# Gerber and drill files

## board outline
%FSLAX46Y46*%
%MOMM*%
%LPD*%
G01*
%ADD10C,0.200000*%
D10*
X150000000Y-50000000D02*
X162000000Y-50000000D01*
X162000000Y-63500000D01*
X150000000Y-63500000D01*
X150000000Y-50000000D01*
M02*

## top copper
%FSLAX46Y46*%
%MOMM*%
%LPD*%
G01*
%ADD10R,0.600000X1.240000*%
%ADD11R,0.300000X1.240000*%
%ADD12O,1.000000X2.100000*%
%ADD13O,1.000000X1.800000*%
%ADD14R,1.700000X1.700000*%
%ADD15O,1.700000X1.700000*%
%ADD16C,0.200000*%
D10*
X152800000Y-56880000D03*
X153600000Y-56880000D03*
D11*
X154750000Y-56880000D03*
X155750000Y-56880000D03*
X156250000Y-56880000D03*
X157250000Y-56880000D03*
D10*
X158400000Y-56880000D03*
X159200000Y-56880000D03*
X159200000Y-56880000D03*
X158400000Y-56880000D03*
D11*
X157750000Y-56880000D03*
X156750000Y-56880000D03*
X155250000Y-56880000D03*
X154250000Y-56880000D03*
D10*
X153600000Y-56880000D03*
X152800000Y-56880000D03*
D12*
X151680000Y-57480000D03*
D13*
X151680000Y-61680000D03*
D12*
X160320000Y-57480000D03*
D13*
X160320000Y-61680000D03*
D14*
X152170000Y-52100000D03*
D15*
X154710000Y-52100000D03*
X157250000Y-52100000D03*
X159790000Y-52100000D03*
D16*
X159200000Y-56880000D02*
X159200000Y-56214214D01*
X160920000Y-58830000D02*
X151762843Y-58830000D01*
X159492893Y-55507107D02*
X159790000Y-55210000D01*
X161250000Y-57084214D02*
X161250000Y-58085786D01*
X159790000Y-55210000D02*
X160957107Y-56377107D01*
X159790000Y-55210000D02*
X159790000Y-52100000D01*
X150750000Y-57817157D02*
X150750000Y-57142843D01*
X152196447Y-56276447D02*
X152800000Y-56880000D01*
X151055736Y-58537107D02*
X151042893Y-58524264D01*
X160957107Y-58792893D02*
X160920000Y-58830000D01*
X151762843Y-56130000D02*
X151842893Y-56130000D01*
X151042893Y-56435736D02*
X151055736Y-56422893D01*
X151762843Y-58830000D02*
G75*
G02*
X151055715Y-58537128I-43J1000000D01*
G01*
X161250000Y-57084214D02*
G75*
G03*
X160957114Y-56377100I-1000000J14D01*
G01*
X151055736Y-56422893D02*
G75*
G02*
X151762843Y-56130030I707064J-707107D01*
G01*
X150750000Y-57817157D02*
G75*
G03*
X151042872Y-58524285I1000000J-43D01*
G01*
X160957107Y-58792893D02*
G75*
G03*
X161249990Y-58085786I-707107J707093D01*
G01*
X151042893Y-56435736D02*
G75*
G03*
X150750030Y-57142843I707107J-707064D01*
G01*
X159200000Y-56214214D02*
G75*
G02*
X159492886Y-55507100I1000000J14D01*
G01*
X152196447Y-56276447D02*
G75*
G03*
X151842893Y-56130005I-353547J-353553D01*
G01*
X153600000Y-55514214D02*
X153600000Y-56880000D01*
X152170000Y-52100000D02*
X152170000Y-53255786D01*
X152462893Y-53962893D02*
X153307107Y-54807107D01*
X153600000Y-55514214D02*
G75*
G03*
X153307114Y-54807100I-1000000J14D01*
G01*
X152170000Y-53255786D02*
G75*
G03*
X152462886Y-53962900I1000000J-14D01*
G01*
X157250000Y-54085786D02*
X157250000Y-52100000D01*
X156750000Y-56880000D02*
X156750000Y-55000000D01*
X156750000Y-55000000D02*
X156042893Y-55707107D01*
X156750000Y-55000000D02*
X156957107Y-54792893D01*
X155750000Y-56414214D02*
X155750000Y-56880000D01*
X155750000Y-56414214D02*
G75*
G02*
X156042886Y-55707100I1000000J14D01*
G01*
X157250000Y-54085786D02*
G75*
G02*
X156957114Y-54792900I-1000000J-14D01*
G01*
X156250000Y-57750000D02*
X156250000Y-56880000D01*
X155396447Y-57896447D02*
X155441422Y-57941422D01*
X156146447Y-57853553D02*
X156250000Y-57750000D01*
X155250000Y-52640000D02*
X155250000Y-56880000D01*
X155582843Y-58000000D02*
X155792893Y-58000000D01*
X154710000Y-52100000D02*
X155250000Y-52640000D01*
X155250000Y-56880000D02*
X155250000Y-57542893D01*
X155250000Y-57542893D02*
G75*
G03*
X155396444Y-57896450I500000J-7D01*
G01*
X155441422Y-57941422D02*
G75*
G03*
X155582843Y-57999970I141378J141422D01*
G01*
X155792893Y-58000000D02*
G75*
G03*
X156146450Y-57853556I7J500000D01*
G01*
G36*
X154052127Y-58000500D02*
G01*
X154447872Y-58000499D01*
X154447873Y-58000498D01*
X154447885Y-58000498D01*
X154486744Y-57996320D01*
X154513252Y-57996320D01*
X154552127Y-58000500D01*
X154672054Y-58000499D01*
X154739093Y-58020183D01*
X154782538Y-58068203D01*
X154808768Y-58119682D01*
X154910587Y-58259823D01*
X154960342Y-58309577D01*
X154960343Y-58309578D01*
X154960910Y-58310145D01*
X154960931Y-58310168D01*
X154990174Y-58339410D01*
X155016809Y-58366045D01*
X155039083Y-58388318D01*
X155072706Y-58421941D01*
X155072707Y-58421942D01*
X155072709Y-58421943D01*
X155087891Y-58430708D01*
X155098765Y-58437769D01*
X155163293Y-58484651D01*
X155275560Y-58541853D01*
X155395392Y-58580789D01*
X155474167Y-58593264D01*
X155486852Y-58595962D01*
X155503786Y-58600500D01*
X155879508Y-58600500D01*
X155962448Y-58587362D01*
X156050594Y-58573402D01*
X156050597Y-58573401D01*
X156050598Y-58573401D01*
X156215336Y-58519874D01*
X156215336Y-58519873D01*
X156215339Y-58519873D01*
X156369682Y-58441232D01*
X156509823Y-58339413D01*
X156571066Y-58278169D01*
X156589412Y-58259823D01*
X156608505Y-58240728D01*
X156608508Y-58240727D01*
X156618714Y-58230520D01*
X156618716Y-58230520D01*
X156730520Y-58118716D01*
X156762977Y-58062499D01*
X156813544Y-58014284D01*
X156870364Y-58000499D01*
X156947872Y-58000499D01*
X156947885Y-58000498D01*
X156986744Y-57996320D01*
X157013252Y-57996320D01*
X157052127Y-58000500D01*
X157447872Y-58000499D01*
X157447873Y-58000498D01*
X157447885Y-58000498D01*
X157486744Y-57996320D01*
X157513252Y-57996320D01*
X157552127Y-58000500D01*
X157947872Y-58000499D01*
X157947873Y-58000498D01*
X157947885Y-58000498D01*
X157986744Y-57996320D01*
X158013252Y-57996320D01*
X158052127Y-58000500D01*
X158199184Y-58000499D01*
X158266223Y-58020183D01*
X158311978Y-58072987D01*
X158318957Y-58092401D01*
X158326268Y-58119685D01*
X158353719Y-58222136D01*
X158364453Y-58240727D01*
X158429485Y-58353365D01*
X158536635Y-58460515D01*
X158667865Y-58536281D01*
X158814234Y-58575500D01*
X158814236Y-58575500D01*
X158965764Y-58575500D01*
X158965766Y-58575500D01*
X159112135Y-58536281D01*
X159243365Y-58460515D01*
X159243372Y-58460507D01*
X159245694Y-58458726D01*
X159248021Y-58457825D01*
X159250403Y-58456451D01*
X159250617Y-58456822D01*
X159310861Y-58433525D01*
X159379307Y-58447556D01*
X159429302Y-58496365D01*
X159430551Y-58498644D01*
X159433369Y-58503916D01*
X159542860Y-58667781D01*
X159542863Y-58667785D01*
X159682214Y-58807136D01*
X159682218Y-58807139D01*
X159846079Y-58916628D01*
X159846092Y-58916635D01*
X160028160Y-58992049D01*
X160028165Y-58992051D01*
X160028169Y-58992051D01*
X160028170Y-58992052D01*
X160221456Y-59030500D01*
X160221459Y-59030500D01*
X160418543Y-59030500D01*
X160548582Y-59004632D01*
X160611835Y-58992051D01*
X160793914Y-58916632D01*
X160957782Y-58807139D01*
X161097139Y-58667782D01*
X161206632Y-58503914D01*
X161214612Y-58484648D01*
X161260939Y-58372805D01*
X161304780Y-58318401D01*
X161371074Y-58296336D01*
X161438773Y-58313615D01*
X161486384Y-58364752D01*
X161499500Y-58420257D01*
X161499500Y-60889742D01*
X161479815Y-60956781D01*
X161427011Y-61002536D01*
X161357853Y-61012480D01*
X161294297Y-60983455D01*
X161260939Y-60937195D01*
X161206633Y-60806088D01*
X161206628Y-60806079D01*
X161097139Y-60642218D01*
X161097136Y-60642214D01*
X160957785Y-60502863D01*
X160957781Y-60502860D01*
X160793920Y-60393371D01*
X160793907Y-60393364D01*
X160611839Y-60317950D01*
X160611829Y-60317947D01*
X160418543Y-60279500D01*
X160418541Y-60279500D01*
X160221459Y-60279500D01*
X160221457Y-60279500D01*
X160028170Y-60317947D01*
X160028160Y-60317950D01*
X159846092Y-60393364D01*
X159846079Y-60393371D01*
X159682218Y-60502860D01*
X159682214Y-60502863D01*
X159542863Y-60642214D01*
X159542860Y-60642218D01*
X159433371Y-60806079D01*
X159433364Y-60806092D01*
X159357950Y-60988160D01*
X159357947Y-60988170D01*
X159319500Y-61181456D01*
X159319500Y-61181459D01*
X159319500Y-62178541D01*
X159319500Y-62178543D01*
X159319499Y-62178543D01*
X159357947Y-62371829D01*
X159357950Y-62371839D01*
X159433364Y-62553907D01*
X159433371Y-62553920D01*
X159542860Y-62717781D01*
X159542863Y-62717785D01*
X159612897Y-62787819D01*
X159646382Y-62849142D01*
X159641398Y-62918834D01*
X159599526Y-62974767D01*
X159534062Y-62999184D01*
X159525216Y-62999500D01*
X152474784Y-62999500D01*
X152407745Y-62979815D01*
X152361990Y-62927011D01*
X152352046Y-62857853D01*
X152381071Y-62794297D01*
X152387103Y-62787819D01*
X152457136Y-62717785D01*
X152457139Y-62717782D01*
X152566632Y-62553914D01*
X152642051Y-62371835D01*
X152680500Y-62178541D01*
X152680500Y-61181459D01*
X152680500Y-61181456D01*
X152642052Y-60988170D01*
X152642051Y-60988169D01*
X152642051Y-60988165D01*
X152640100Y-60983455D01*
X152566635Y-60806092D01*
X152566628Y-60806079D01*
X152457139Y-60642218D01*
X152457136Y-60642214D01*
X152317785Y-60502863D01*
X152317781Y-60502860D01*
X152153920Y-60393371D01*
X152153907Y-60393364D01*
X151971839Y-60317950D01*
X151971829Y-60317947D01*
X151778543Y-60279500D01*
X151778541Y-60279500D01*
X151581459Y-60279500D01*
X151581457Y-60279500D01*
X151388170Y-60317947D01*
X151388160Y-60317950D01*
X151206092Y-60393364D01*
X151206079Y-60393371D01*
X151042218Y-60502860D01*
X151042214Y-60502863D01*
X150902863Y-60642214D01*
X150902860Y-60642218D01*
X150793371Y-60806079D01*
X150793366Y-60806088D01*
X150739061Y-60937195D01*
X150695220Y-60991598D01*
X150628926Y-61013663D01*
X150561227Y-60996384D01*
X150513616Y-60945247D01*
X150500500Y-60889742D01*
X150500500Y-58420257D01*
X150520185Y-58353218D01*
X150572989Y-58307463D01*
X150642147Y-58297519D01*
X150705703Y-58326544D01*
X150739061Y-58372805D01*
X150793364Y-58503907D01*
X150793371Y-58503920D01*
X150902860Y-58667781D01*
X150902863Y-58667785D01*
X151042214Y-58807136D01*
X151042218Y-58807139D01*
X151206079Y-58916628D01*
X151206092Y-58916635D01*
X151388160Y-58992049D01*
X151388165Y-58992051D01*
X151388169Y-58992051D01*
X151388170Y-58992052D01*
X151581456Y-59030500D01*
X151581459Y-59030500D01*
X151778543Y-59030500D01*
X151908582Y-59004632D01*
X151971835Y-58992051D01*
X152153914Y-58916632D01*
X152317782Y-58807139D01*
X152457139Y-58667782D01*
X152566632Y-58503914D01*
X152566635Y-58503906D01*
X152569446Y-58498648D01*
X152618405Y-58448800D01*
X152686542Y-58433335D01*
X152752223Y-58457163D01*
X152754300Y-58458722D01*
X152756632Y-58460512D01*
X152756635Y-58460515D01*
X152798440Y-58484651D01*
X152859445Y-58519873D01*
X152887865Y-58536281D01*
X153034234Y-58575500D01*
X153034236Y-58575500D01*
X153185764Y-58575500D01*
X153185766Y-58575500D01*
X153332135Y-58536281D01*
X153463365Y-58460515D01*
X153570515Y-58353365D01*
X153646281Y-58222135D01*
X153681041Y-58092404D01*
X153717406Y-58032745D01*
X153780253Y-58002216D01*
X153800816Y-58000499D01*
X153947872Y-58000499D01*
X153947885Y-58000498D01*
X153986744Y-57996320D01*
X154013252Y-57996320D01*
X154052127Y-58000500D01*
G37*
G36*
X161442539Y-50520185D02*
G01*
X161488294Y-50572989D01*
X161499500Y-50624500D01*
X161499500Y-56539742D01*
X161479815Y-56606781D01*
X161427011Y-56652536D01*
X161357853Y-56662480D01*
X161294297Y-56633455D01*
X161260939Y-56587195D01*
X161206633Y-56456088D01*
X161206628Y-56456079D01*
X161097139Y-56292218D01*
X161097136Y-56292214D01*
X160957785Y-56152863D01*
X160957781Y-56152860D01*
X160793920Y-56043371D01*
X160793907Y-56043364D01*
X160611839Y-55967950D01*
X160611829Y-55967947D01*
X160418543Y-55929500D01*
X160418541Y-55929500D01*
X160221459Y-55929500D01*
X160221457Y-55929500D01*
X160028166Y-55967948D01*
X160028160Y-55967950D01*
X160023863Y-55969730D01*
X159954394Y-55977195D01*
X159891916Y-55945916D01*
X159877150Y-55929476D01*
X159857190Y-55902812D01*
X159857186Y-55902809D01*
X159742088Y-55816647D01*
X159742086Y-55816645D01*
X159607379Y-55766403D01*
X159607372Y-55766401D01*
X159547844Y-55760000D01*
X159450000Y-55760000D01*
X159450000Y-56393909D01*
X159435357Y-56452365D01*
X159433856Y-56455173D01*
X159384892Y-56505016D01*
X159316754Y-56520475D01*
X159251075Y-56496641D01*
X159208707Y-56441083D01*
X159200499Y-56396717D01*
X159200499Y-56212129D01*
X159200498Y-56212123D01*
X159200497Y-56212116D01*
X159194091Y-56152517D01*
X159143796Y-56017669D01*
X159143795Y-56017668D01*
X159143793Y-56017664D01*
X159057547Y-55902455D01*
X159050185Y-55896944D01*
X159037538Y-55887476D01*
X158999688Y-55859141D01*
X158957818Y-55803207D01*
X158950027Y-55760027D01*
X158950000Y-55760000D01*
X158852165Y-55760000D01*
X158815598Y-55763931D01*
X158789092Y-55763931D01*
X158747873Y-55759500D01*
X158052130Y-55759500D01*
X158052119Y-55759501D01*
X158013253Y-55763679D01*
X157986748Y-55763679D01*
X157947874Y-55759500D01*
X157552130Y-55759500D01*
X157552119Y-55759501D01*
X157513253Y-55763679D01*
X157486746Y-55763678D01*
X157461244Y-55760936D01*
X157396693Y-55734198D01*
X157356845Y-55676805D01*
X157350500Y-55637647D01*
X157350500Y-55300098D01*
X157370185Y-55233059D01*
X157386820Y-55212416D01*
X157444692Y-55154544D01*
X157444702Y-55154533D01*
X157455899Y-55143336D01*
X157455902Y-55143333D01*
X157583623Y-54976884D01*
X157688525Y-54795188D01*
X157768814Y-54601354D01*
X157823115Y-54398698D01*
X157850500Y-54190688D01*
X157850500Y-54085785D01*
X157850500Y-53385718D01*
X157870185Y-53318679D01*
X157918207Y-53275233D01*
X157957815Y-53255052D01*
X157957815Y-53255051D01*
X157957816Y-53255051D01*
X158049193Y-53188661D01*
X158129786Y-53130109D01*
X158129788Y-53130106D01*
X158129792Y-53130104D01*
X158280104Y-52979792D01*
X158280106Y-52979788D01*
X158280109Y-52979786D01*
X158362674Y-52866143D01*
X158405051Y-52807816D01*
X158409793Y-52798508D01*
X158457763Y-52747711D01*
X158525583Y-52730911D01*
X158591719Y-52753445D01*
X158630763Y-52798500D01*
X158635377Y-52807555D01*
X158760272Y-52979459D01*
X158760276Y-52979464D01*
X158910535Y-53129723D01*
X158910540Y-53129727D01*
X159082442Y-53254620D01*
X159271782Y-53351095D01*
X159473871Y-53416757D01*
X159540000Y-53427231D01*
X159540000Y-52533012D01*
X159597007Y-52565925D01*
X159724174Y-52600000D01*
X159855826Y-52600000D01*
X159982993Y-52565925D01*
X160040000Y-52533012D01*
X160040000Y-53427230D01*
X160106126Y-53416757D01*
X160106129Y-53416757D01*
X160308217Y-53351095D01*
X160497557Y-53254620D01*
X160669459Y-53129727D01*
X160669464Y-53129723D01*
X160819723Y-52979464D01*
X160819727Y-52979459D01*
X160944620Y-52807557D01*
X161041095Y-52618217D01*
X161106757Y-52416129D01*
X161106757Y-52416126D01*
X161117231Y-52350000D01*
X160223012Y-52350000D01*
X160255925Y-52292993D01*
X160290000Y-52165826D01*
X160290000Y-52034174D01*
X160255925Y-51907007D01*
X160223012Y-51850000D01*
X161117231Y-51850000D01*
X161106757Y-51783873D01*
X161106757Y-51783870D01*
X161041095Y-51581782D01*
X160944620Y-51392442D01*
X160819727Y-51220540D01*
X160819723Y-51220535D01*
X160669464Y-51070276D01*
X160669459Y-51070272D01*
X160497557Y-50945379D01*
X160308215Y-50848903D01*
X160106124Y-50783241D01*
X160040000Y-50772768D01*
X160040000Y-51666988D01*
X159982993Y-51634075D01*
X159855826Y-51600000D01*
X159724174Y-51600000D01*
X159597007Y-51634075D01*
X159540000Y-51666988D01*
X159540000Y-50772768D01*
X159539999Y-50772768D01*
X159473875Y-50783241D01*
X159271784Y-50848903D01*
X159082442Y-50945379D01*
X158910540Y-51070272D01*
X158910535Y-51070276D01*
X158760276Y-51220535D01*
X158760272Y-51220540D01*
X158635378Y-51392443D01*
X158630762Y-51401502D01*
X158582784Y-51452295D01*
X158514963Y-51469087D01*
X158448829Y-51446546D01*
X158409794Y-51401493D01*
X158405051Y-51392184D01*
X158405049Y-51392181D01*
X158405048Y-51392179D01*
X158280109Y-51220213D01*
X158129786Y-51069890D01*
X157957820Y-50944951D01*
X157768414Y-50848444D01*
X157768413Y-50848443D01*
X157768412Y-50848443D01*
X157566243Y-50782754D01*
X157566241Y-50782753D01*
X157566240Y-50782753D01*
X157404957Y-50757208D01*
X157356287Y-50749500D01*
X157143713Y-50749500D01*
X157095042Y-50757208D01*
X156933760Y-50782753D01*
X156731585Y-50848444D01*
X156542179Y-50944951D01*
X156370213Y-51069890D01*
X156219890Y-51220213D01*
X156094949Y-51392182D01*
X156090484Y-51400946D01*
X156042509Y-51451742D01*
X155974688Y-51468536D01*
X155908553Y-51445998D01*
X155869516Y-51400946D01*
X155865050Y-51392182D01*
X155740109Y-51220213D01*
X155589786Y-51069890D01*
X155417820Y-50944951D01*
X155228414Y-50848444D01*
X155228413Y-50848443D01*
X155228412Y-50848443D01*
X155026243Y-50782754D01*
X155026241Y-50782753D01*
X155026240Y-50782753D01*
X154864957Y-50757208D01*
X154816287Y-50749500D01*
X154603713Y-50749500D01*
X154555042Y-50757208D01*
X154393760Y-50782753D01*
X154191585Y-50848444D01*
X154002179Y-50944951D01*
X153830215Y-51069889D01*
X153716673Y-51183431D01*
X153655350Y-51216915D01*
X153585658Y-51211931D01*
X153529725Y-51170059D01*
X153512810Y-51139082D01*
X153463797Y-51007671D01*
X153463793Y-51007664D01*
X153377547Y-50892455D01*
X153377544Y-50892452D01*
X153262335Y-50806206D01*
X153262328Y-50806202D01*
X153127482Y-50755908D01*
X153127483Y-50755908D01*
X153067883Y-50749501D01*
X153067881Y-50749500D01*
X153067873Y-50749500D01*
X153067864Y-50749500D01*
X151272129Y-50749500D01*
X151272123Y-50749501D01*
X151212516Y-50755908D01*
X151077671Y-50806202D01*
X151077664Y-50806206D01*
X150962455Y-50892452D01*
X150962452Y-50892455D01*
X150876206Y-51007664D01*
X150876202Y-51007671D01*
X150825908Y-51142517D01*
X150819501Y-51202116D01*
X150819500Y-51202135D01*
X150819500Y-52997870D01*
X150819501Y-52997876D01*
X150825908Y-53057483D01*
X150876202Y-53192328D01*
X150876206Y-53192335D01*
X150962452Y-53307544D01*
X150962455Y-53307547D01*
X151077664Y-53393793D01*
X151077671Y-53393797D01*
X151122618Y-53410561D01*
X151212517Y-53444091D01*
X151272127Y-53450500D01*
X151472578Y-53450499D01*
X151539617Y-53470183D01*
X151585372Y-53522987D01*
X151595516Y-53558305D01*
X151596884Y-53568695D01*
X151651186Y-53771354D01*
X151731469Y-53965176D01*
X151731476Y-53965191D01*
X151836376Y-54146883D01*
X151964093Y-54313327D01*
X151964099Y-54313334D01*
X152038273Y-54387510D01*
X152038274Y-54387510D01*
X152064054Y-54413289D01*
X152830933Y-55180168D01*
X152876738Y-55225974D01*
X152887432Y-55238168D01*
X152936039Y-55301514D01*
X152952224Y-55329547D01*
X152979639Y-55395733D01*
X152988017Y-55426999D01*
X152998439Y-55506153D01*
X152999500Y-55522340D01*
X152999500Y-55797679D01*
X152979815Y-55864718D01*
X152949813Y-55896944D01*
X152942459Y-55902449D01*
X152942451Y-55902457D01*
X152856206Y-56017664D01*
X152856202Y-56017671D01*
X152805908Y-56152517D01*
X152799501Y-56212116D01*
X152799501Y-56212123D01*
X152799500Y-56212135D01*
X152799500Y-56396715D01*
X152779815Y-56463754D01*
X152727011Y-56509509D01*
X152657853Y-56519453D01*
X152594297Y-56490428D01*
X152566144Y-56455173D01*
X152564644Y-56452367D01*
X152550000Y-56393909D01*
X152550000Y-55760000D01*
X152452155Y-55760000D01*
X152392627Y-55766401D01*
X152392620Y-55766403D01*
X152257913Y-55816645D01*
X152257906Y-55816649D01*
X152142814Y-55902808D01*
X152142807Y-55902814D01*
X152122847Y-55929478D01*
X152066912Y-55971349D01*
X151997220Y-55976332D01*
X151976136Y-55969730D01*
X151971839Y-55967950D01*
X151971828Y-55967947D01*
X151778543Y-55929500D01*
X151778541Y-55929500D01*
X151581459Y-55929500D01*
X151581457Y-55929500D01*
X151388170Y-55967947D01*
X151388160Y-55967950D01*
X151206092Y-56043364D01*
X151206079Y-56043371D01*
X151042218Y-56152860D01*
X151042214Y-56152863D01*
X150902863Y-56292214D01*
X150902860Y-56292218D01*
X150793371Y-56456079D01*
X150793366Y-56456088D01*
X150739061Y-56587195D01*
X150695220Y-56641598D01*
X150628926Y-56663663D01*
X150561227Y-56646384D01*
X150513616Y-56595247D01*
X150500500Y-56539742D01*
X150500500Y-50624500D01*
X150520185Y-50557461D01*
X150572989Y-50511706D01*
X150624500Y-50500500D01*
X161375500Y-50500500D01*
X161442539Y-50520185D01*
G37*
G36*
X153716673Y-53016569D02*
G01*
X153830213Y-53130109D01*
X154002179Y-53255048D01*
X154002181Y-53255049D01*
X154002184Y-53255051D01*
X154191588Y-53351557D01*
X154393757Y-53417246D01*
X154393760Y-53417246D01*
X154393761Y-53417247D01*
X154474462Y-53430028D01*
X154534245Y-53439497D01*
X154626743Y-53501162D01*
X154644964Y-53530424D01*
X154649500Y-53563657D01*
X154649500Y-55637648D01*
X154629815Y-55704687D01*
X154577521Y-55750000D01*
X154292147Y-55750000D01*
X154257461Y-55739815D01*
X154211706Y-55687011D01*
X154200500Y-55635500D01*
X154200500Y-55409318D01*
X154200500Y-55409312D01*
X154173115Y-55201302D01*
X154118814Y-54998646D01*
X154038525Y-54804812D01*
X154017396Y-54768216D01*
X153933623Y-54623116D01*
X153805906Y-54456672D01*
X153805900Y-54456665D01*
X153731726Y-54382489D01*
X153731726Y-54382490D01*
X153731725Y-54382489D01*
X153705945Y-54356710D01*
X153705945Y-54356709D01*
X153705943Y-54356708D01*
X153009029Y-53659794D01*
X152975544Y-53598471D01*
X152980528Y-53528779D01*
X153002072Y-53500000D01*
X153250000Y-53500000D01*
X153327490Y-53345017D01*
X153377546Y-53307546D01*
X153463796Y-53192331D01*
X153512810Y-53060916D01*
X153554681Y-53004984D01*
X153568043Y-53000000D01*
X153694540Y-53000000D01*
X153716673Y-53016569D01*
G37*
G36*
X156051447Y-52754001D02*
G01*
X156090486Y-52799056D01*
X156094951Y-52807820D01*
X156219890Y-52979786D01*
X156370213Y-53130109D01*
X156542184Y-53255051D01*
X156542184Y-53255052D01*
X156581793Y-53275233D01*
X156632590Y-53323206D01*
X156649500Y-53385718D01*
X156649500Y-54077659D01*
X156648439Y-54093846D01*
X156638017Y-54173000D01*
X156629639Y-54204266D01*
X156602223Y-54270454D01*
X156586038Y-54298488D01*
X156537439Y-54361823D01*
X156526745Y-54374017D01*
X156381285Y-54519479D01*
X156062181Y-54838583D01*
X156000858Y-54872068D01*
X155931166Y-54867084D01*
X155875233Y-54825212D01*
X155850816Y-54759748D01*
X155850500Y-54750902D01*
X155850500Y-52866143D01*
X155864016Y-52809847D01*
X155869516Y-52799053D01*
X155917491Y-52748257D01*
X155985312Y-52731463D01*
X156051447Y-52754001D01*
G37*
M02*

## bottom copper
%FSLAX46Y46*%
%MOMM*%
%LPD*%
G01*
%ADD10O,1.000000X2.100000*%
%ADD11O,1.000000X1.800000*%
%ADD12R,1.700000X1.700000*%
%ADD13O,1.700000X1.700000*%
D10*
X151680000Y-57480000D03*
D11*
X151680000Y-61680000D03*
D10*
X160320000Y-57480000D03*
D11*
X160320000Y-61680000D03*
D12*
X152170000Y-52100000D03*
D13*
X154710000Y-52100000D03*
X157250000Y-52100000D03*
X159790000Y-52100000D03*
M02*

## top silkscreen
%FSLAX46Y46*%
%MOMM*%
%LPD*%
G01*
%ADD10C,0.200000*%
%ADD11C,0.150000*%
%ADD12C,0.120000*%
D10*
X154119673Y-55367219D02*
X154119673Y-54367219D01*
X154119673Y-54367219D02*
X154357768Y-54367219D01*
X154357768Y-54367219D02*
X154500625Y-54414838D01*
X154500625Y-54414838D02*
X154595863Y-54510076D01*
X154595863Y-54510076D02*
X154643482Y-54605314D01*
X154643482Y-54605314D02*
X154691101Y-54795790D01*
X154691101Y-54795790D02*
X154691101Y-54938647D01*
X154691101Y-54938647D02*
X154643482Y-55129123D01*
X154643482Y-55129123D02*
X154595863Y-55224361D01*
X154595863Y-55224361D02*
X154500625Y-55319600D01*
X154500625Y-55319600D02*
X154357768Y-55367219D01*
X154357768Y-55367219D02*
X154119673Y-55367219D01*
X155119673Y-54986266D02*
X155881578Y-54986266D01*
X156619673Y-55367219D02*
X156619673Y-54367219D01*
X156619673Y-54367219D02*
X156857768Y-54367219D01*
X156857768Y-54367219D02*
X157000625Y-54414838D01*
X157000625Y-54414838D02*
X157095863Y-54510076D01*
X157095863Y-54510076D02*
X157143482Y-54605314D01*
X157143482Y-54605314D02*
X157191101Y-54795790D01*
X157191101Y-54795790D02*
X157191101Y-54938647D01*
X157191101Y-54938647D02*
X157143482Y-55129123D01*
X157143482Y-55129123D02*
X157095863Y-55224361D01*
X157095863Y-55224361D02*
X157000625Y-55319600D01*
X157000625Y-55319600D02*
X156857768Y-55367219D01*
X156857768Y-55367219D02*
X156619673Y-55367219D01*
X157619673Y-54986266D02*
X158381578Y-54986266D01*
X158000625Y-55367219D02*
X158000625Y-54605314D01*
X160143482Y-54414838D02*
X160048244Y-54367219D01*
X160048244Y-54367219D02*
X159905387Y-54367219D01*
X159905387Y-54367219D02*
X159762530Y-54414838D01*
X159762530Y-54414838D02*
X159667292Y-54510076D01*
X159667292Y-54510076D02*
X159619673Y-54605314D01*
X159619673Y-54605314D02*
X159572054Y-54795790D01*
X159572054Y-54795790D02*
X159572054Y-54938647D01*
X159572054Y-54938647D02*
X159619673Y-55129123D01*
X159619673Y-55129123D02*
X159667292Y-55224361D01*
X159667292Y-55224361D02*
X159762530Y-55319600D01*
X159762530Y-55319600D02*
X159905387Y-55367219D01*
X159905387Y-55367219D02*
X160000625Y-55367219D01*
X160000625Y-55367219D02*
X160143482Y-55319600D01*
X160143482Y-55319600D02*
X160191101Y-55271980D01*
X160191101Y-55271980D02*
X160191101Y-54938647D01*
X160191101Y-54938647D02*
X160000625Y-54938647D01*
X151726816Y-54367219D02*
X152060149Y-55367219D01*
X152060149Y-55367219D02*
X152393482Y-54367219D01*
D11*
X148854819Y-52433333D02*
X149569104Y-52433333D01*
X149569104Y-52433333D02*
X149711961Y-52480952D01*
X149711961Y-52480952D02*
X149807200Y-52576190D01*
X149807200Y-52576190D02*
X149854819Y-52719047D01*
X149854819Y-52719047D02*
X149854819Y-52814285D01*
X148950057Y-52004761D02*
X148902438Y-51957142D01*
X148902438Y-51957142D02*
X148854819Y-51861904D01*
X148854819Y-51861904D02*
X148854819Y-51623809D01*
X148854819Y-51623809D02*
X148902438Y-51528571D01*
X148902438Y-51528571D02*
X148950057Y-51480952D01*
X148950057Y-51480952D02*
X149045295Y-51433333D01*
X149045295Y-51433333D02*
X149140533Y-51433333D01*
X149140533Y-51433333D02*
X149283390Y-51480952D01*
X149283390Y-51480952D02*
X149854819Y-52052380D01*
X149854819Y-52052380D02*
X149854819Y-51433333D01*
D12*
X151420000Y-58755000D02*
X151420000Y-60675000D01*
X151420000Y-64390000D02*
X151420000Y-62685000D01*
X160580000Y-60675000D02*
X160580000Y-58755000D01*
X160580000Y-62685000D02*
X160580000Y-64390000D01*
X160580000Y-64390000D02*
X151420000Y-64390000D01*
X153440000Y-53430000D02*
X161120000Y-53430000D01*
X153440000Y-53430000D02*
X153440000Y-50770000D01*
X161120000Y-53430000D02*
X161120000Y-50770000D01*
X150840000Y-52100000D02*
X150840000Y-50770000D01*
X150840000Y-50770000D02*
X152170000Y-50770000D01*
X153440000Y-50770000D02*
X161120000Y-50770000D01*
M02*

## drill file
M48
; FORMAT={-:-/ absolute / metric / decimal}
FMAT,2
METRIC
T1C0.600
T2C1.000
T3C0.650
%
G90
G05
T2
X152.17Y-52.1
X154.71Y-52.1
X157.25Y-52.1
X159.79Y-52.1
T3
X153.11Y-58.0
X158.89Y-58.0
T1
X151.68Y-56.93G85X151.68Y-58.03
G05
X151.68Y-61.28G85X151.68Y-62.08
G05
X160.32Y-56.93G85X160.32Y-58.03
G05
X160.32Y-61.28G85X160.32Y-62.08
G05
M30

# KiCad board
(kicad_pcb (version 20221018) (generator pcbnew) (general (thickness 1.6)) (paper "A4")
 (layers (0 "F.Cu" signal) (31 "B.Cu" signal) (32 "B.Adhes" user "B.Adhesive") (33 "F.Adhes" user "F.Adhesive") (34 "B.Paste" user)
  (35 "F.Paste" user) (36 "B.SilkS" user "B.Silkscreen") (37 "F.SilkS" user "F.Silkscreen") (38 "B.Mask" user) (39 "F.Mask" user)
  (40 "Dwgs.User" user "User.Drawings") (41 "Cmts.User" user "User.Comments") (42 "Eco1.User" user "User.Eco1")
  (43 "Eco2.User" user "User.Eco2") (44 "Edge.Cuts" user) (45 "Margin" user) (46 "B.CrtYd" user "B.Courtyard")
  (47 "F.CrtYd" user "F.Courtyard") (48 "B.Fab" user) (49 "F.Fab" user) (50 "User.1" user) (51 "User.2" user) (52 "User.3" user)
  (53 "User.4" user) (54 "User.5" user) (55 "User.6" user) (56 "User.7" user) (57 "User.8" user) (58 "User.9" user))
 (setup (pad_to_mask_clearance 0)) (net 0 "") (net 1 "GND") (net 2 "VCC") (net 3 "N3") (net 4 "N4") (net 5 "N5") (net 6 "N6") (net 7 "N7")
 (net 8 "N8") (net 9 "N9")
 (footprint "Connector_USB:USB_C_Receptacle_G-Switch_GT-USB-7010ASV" (layer "F.Cu") (at 156 60.605)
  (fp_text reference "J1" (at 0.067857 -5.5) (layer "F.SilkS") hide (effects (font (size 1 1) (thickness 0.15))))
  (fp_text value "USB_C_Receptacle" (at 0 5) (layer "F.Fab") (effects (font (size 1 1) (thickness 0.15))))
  (fp_line (start -4.58 -1.85) (end -4.58 0.07) (stroke (width 0.12) (type solid)) (layer "F.SilkS"))
  (fp_line (start -4.58 3.785) (end -4.58 2.08) (stroke (width 0.12) (type solid)) (layer "F.SilkS"))
  (fp_line (start 4.58 0.07) (end 4.58 -1.85) (stroke (width 0.12) (type solid)) (layer "F.SilkS"))
  (fp_line (start 4.58 2.08) (end 4.58 3.785) (stroke (width 0.12) (type solid)) (layer "F.SilkS"))
  (fp_line (start 4.58 3.785) (end -4.58 3.785) (stroke (width 0.12) (type solid)) (layer "F.SilkS"))
  (pad "" np_thru_hole circle (at -2.89 -2.605) (size 0.65 0.65) (drill 0.65) (layers "*.Cu" "*.Mask"))
  (pad "" np_thru_hole circle (at 2.89 -2.605) (size 0.65 0.65) (drill 0.65) (layers "*.Cu" "*.Mask"))
  (pad "A1" smd rect (at -3.2 -3.725) (size 0.6 1.24) (layers "F.Cu" "F.Paste" "F.Mask") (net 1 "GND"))
  (pad "A4" smd rect (at -2.4 -3.725) (size 0.6 1.24) (layers "F.Cu" "F.Paste" "F.Mask") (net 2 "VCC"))
  (pad "A5" smd rect (at -1.25 -3.725) (size 0.3 1.24) (layers "F.Cu" "F.Paste" "F.Mask") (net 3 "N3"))
  (pad "A6" smd rect (at -0.25 -3.725) (size 0.3 1.24) (layers "F.Cu" "F.Paste" "F.Mask") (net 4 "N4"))
  (pad "A7" smd rect (at 0.25 -3.725) (size 0.3 1.24) (layers "F.Cu" "F.Paste" "F.Mask") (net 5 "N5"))
  (pad "A8" smd rect (at 1.25 -3.725) (size 0.3 1.24) (layers "F.Cu" "F.Paste" "F.Mask") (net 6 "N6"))
  (pad "A9" smd rect (at 2.4 -3.725) (size 0.6 1.24) (layers "F.Cu" "F.Paste" "F.Mask") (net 2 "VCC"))
  (pad "A12" smd rect (at 3.2 -3.725) (size 0.6 1.24) (layers "F.Cu" "F.Paste" "F.Mask") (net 1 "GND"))
  (pad "B1" smd rect (at 3.2 -3.725) (size 0.6 1.24) (layers "F.Cu" "F.Paste" "F.Mask") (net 1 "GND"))
  (pad "B4" smd rect (at 2.4 -3.725) (size 0.6 1.24) (layers "F.Cu" "F.Paste" "F.Mask") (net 2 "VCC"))
  (pad "B5" smd rect (at 1.75 -3.725) (size 0.3 1.24) (layers "F.Cu" "F.Paste" "F.Mask") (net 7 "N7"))
  (pad "B6" smd rect (at 0.75 -3.725) (size 0.3 1.24) (layers "F.Cu" "F.Paste" "F.Mask") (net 4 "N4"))
  (pad "B7" smd rect (at -0.75 -3.725) (size 0.3 1.24) (layers "F.Cu" "F.Paste" "F.Mask") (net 5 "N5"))
  (pad "B8" smd rect (at -1.75 -3.725) (size 0.3 1.24) (layers "F.Cu" "F.Paste" "F.Mask") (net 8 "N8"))
  (pad "B9" smd rect (at -2.4 -3.725) (size 0.6 1.24) (layers "F.Cu" "F.Paste" "F.Mask") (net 2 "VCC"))
  (pad "B12" smd rect (at -3.2 -3.725) (size 0.6 1.24) (layers "F.Cu" "F.Paste" "F.Mask") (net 1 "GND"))
  (pad "S1" thru_hole oval (at -4.32 -3.125) (size 1 2.1) (drill oval 0.6 1.7) (layers "*.Cu" "*.Mask") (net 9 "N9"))
  (pad "S1" thru_hole oval (at -4.32 1.075) (size 1 1.8) (drill oval 0.6 1.4) (layers "*.Cu" "*.Mask") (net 9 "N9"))
  (pad "S1" thru_hole oval (at 4.32 -3.125) (size 1 2.1) (drill oval 0.6 1.7) (layers "*.Cu" "*.Mask") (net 9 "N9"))
  (pad "S1" thru_hole oval (at 4.32 1.075) (size 1 1.8) (drill oval 0.6 1.4) (layers "*.Cu" "*.Mask") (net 9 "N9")))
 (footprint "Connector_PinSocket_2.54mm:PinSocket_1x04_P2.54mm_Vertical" (layer "F.Cu") (at 152.17 52.1 90)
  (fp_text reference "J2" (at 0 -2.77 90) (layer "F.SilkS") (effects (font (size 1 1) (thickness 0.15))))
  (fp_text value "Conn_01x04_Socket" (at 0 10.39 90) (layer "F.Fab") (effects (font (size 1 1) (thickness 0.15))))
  (fp_line (start -1.33 1.27) (end -1.33 8.95) (stroke (width 0.12) (type solid)) (layer "F.SilkS"))
  (fp_line (start -1.33 1.27) (end 1.33 1.27) (stroke (width 0.12) (type solid)) (layer "F.SilkS"))
  (fp_line (start -1.33 8.95) (end 1.33 8.95) (stroke (width 0.12) (type solid)) (layer "F.SilkS"))
  (fp_line (start 0 -1.33) (end 1.33 -1.33) (stroke (width 0.12) (type solid)) (layer "F.SilkS"))
  (fp_line (start 1.33 -1.33) (end 1.33 0) (stroke (width 0.12) (type solid)) (layer "F.SilkS"))
  (fp_line (start 1.33 1.27) (end 1.33 8.95) (stroke (width 0.12) (type solid)) (layer "F.SilkS"))
  (pad "1" thru_hole rect (at 0 0 90) (size 1.7 1.7) (drill 1) (layers "*.Cu" "*.Mask") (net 2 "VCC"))
  (pad "2" thru_hole oval (at 0 2.54 90) (size 1.7 1.7) (drill 1) (layers "*.Cu" "*.Mask") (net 5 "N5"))
  (pad "3" thru_hole oval (at 0 5.08 90) (size 1.7 1.7) (drill 1) (layers "*.Cu" "*.Mask") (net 4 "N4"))
  (pad "4" thru_hole oval (at 0 7.62 90) (size 1.7 1.7) (drill 1) (layers "*.Cu" "*.Mask") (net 1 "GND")))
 (gr_rect locked (start 150 50) (end 162 63.5) (stroke (width 0.2) (type solid)) (fill none) (layer "Edge.Cuts"))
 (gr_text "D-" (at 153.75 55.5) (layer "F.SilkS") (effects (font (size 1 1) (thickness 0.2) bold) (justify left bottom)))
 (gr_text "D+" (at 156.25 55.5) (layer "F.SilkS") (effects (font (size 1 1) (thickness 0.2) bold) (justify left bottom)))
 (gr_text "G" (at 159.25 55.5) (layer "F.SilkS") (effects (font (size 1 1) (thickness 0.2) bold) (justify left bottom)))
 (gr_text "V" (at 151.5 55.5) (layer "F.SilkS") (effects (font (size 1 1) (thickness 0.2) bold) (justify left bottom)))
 (segment (start 159.2 56.88) (end 159.2 56.214214) (width 0.2) (layer "F.Cu") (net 1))
 (segment (start 160.92 58.83) (end 151.762843 58.83) (width 0.2) (layer "F.Cu") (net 1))
 (segment (start 159.492893 55.507107) (end 159.79 55.21) (width 0.2) (layer "F.Cu") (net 1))
 (segment (start 161.25 57.084214) (end 161.25 58.085786) (width 0.2) (layer "F.Cu") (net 1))
 (segment (start 159.79 55.21) (end 160.957107 56.377107) (width 0.2) (layer "F.Cu") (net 1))
 (segment (start 159.79 55.21) (end 159.79 52.1) (width 0.2) (layer "F.Cu") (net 1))
 (segment (start 150.75 57.817157) (end 150.75 57.142843) (width 0.2) (layer "F.Cu") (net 1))
 (segment (start 152.196447 56.276447) (end 152.8 56.88) (width 0.2) (layer "F.Cu") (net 1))
 (segment (start 151.055736 58.537107) (end 151.042893 58.524264) (width 0.2) (layer "F.Cu") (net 1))
 (segment (start 160.957107 58.792893) (end 160.92 58.83) (width 0.2) (layer "F.Cu") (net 1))
 (segment (start 151.762843 56.13) (end 151.842893 56.13) (width 0.2) (layer "F.Cu") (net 1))
 (segment (start 151.042893 56.435736) (end 151.055736 56.422893) (width 0.2) (layer "F.Cu") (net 1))
 (arc (start 151.762843 58.83) (mid 151.38016 58.75388) (end 151.055736 58.537107) (width 0.2) (layer "F.Cu") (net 1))
 (arc (start 161.25 57.084214) (mid 161.17388 56.701531) (end 160.957107 56.377107) (width 0.2) (layer "F.Cu") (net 1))
 (arc (start 151.055736 56.422893) (mid 151.380159 56.20612) (end 151.762843 56.13) (width 0.2) (layer "F.Cu") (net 1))
 (arc (start 150.75 57.817157) (mid 150.82612 58.19984) (end 151.042893 58.524264) (width 0.2) (layer "F.Cu") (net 1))
 (arc (start 160.957107 58.792893) (mid 161.17388 58.46847) (end 161.25 58.085786) (width 0.2) (layer "F.Cu") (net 1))
 (arc (start 151.042893 56.435736) (mid 150.82612 56.760159) (end 150.75 57.142843) (width 0.2) (layer "F.Cu") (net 1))
 (arc (start 159.2 56.214214) (mid 159.27612 55.831531) (end 159.492893 55.507107) (width 0.2) (layer "F.Cu") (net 1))
 (arc (start 152.196447 56.276447) (mid 152.034235 56.16806) (end 151.842893 56.13) (width 0.2) (layer "F.Cu") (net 1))
 (segment (start 153.6 55.514214) (end 153.6 56.88) (width 0.2) (layer "F.Cu") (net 2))
 (segment (start 152.17 52.1) (end 152.17 53.255786) (width 0.2) (layer "F.Cu") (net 2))
 (segment (start 152.462893 53.962893) (end 153.307107 54.807107) (width 0.2) (layer "F.Cu") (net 2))
 (arc (start 153.6 55.514214) (mid 153.52388 55.131531) (end 153.307107 54.807107) (width 0.2) (layer "F.Cu") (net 2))
 (arc (start 152.17 53.255786) (mid 152.24612 53.638469) (end 152.462893 53.962893) (width 0.2) (layer "F.Cu") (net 2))
 (segment (start 157.25 54.085786) (end 157.25 52.1) (width 0.2) (layer "F.Cu") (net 4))
 (segment (start 156.75 56.88) (end 156.75 55) (width 0.2) (layer "F.Cu") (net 4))
 (segment (start 156.75 55) (end 156.042893 55.707107) (width 0.2) (layer "F.Cu") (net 4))
 (segment (start 156.75 55) (end 156.957107 54.792893) (width 0.2) (layer "F.Cu") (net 4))
 (segment (start 155.75 56.414214) (end 155.75 56.88) (width 0.2) (layer "F.Cu") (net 4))
 (arc (start 155.75 56.414214) (mid 155.82612 56.031531) (end 156.042893 55.707107) (width 0.2) (layer "F.Cu") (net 4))
 (arc (start 157.25 54.085786) (mid 157.17388 54.468469) (end 156.957107 54.792893) (width 0.2) (layer "F.Cu") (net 4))
 (segment (start 156.25 57.75) (end 156.25 56.88) (width 0.2) (layer "F.Cu") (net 5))
 (segment (start 155.396447 57.896447) (end 155.441422 57.941422) (width 0.2) (layer "F.Cu") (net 5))
 (segment (start 156.146447 57.853553) (end 156.25 57.75) (width 0.2) (layer "F.Cu") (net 5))
 (segment (start 155.25 52.64) (end 155.25 56.88) (width 0.2) (layer "F.Cu") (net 5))
 (segment (start 155.582843 58) (end 155.792893 58) (width 0.2) (layer "F.Cu") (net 5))
 (segment (start 154.71 52.1) (end 155.25 52.64) (width 0.2) (layer "F.Cu") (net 5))
 (segment (start 155.25 56.88) (end 155.25 57.542893) (width 0.2) (layer "F.Cu") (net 5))
 (arc (start 155.25 57.542893) (mid 155.28806 57.734235) (end 155.396447 57.896447) (width 0.2) (layer "F.Cu") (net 5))
 (arc (start 155.441422 57.941422) (mid 155.506307 57.984776) (end 155.582843 58) (width 0.2) (layer "F.Cu") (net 5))
 (arc (start 155.792893 58) (mid 155.984235 57.96194) (end 156.146447 57.853553) (width 0.2) (layer "F.Cu") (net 5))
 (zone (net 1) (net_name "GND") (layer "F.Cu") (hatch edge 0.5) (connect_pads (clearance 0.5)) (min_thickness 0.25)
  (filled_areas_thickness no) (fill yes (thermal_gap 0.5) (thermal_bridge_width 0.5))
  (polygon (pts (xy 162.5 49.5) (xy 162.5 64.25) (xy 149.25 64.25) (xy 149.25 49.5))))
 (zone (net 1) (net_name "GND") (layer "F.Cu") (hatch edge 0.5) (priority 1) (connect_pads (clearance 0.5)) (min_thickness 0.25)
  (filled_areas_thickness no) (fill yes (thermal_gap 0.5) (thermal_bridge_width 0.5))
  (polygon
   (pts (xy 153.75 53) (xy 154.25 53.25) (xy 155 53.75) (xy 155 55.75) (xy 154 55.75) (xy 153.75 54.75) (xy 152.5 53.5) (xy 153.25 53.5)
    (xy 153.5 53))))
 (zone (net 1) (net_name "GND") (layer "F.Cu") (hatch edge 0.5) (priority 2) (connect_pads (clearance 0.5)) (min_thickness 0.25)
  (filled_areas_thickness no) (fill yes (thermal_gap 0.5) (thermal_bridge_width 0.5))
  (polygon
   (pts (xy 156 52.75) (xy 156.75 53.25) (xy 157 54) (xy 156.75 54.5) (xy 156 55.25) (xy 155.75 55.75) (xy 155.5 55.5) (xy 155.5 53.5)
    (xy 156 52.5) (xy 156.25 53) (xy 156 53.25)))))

